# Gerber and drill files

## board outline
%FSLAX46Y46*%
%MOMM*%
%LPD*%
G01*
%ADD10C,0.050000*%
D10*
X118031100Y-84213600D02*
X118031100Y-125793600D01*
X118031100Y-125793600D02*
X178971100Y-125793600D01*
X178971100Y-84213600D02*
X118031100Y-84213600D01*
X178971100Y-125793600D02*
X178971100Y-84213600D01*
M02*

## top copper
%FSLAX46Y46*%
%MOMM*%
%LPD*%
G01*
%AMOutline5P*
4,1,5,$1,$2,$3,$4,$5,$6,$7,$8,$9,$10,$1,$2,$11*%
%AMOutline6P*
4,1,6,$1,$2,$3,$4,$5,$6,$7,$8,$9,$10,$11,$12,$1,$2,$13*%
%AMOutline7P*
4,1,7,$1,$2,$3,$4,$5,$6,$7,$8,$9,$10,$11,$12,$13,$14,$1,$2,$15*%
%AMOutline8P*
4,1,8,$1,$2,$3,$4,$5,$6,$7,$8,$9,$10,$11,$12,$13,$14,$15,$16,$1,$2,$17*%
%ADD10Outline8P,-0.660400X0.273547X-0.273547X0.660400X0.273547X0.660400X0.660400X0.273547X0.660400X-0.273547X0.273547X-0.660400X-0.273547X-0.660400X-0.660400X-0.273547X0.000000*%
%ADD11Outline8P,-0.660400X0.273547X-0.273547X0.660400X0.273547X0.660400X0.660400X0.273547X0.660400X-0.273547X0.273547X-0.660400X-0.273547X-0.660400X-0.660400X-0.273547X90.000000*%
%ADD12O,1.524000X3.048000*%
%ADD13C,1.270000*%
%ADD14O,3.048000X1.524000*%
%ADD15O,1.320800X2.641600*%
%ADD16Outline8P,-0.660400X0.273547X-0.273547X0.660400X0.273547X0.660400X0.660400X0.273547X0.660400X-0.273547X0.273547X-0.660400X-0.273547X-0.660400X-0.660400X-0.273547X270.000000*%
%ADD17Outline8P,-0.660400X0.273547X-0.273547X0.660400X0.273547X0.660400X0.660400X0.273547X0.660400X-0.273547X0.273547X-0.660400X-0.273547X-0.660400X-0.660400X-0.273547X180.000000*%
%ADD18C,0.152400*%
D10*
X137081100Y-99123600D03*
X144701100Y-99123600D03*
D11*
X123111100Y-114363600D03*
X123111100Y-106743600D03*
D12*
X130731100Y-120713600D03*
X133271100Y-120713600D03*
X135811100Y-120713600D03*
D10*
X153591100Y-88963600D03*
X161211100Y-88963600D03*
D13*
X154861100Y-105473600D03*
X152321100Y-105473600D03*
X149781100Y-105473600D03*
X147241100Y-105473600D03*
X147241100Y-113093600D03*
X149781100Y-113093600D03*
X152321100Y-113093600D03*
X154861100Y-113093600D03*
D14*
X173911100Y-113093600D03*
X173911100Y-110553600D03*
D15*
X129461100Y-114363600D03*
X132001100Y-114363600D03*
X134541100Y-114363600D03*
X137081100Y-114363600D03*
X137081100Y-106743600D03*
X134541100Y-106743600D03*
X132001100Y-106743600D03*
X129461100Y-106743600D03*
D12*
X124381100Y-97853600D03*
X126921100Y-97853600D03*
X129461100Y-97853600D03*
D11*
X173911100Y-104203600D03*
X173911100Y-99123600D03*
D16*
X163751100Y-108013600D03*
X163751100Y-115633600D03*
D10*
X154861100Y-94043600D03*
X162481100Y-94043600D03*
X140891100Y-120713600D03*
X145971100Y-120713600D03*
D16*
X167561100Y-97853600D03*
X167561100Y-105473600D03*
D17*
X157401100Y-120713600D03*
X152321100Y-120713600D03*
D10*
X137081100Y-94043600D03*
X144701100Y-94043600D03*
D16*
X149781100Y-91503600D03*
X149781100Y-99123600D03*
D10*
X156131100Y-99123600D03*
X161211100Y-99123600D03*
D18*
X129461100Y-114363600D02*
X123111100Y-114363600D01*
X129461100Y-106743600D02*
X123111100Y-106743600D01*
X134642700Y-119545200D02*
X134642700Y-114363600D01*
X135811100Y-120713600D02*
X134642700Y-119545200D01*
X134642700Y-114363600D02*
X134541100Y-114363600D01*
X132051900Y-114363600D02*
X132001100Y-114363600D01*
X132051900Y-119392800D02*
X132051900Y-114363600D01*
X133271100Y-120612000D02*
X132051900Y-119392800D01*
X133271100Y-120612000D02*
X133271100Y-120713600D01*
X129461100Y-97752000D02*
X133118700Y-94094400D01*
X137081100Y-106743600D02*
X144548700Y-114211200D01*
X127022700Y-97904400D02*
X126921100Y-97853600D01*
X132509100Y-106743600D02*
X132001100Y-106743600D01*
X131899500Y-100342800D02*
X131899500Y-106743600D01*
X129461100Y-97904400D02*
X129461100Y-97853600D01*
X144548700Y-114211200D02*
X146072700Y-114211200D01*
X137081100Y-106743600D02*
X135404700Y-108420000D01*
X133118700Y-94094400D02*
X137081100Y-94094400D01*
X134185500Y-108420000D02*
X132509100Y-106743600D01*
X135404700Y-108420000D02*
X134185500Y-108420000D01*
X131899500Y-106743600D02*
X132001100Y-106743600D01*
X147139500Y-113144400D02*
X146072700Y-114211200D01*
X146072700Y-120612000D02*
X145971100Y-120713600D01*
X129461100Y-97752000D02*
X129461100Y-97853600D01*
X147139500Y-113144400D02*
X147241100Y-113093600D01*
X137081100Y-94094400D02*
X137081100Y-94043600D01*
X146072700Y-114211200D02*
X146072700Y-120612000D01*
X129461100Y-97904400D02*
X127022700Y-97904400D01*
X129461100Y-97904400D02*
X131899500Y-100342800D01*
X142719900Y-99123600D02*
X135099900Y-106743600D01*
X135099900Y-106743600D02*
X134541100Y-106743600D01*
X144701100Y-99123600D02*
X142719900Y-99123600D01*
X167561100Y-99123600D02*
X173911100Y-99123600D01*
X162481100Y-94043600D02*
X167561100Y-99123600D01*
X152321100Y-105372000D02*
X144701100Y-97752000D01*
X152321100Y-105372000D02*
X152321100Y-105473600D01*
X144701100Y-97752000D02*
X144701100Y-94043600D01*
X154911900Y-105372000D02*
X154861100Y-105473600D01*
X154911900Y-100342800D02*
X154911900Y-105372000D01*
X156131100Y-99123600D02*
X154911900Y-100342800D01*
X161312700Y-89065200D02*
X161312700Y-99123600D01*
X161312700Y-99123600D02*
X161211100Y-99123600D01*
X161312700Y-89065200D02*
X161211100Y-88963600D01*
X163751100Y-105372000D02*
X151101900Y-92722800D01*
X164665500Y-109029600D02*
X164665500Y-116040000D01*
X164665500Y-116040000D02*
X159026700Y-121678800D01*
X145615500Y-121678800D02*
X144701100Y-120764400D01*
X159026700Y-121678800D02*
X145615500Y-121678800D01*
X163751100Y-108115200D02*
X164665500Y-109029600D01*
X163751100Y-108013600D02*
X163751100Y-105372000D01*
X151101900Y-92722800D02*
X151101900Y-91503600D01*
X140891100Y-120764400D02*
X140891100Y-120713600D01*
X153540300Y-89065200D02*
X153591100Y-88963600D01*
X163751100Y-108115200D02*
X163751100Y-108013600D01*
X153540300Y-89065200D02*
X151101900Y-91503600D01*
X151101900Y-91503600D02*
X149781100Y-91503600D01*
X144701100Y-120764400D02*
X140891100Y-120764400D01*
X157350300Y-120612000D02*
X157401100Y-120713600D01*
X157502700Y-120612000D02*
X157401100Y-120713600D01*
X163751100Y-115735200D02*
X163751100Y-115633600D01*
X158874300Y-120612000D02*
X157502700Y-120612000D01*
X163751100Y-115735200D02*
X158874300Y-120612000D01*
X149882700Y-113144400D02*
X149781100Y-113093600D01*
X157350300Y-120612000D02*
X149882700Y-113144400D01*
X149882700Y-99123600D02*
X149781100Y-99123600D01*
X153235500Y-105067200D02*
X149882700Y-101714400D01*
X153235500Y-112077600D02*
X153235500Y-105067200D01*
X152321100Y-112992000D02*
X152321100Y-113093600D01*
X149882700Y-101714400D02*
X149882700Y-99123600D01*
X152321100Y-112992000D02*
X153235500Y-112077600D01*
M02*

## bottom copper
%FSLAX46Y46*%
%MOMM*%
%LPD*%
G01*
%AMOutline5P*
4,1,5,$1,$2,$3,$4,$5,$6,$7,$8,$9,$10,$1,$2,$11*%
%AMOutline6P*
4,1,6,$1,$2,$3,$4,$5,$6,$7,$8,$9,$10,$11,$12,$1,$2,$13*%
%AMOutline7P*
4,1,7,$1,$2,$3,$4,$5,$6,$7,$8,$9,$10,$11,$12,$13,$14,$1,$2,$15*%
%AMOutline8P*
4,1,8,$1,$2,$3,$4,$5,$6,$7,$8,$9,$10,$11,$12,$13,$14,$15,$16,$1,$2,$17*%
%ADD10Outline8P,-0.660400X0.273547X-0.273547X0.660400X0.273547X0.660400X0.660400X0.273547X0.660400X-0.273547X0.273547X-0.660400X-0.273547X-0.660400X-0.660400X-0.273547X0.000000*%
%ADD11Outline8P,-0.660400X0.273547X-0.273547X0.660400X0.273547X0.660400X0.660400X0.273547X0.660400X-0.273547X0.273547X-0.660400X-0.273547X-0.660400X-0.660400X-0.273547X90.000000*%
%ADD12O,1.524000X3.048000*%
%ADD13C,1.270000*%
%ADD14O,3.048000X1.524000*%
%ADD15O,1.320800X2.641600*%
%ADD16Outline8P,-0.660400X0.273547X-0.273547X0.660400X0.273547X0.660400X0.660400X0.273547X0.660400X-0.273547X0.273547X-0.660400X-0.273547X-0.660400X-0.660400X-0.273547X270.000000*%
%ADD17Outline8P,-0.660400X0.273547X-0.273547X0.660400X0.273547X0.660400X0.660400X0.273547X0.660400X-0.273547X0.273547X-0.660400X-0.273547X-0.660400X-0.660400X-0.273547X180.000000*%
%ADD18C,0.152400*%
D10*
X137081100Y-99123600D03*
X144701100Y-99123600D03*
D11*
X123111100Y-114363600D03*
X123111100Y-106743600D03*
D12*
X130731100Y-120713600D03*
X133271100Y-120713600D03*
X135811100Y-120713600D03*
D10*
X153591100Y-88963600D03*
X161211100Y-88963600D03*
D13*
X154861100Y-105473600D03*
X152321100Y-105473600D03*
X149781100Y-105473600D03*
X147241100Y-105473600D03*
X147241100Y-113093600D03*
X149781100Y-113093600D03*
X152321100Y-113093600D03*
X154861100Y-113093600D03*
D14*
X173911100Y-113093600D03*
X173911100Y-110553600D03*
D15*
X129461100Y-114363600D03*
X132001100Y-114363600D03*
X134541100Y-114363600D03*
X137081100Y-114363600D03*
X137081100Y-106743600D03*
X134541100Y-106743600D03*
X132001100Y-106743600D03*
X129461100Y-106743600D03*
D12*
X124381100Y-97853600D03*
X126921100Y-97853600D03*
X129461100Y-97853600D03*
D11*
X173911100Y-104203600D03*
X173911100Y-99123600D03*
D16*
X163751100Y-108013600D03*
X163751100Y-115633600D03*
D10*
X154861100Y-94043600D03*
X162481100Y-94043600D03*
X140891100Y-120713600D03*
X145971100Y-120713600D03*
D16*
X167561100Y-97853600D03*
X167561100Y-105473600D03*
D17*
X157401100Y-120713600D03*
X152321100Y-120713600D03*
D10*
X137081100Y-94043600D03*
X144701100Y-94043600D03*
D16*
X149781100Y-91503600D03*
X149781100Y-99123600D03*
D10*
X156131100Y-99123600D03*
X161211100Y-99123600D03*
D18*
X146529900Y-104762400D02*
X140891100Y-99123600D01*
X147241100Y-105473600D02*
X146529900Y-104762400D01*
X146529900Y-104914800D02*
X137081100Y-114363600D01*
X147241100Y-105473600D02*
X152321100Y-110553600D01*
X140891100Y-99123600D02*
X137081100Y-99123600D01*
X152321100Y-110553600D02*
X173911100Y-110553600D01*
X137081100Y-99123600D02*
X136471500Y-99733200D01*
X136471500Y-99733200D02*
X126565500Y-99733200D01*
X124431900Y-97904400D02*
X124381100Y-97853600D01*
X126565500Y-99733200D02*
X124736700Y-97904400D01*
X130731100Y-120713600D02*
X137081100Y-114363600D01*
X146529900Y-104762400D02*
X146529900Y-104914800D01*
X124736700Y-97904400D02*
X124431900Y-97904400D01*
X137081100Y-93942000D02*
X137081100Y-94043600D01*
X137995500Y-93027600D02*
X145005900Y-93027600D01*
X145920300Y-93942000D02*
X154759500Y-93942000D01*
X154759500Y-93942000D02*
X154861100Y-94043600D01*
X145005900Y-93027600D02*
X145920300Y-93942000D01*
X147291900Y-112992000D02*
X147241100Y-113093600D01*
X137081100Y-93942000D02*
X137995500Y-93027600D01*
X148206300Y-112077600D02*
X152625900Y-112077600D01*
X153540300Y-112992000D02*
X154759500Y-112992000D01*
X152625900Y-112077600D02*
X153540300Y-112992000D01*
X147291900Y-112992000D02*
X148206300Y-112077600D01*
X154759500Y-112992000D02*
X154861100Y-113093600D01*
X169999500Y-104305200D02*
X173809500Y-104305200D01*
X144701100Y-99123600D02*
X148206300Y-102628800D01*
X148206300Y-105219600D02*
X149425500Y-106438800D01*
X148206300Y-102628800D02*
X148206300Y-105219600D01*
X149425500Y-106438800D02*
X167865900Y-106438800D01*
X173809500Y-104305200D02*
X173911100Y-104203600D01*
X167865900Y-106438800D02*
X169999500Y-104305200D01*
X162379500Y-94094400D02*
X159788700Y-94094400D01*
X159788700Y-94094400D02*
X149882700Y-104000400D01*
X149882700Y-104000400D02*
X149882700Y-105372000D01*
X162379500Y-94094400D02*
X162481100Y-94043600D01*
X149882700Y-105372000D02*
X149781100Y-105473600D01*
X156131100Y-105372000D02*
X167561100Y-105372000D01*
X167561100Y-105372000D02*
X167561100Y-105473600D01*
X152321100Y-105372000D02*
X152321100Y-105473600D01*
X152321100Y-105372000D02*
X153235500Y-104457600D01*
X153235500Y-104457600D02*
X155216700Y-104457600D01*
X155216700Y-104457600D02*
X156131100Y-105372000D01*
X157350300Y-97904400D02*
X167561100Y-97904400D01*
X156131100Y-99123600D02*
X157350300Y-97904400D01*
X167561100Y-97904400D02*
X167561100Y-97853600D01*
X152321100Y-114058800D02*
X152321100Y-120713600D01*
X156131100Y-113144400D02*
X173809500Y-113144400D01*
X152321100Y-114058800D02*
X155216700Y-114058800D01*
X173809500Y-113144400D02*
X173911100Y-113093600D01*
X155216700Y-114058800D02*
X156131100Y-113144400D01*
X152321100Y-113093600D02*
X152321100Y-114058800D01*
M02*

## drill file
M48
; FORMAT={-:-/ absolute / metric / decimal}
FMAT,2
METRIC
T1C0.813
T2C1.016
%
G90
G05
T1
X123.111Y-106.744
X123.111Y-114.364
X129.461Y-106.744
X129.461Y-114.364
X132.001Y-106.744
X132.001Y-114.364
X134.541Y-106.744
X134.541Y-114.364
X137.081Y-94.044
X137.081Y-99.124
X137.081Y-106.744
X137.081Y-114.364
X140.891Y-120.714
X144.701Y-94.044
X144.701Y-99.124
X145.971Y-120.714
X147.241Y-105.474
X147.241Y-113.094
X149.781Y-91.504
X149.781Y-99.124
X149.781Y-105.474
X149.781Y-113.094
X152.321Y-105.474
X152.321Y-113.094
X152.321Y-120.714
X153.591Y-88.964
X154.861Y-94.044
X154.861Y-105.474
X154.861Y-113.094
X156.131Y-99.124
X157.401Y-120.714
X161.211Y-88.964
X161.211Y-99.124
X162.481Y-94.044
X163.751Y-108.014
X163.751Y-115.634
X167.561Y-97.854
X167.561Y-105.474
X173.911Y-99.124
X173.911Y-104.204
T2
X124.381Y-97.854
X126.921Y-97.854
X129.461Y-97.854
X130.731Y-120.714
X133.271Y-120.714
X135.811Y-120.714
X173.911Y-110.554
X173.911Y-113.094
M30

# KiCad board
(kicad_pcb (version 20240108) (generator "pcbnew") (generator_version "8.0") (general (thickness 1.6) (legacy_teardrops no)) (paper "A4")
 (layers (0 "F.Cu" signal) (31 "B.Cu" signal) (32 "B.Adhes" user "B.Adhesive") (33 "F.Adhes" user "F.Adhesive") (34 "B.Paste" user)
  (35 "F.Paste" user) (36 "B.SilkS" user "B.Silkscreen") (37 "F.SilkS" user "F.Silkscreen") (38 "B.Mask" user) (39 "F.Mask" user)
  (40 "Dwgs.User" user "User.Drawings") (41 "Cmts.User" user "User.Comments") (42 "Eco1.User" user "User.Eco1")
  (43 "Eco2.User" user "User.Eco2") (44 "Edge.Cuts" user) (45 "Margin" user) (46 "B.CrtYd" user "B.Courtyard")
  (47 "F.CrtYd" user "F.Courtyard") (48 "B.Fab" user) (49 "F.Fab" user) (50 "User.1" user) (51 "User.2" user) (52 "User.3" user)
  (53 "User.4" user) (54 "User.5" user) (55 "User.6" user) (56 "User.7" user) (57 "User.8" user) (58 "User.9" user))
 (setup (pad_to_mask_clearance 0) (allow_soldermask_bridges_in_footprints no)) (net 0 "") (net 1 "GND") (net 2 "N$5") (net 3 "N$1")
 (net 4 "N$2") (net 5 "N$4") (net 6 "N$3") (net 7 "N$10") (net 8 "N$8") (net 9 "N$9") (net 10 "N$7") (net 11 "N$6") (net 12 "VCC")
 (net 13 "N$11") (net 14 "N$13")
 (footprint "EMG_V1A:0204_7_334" (layer "F.Cu") (at 140.8911 99.1236)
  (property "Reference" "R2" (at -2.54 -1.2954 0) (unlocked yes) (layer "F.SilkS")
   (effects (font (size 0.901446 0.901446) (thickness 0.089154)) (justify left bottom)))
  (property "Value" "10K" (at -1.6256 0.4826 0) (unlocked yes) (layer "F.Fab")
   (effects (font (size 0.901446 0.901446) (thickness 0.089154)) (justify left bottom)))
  (pad "1" thru_hole roundrect (at -3.81 0) (size 1.3208 1.3208) (drill 0.8128) (layers "*.Cu" "*.Mask") (remove_unused_layers no)
   (roundrect_rratio 0.25) (chamfer_ratio 0.2928932188) (chamfer top_left top_right bottom_left bottom_right) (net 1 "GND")
   (solder_mask_margin 0.1016) (thermal_bridge_angle 0))
  (pad "2" thru_hole roundrect (at 3.81 0) (size 1.3208 1.3208) (drill 0.8128) (layers "*.Cu" "*.Mask") (remove_unused_layers no)
   (roundrect_rratio 0.25) (chamfer_ratio 0.2928932188) (chamfer top_left top_right bottom_left bottom_right) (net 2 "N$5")
   (solder_mask_margin 0.1016) (thermal_bridge_angle 0)))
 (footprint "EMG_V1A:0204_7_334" (layer "F.Cu") (at 123.1111 110.5536 90)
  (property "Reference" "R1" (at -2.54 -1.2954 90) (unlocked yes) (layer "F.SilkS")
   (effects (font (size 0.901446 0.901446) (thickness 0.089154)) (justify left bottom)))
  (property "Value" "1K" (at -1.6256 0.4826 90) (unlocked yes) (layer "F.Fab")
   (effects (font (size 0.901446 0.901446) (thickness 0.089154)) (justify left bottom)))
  (pad "1" thru_hole roundrect (at -3.81 0 90) (size 1.3208 1.3208) (drill 0.8128) (layers "*.Cu" "*.Mask") (remove_unused_layers no)
   (roundrect_rratio 0.25) (chamfer_ratio 0.2928932188) (chamfer top_left top_right bottom_left bottom_right) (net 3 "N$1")
   (solder_mask_margin 0.1016) (thermal_bridge_angle 0))
  (pad "2" thru_hole roundrect (at 3.81 0 90) (size 1.3208 1.3208) (drill 0.8128) (layers "*.Cu" "*.Mask") (remove_unused_layers no)
   (roundrect_rratio 0.25) (chamfer_ratio 0.2928932188) (chamfer top_left top_right bottom_left bottom_right) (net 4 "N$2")
   (solder_mask_margin 0.1016) (thermal_bridge_angle 0)))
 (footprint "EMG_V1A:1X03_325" (layer "F.Cu") (at 133.2711 120.7136)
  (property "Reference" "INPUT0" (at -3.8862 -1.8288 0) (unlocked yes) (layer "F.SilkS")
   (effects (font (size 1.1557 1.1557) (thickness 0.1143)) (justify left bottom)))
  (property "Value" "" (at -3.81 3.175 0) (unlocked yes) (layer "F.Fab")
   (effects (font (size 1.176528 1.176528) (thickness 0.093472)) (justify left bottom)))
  (pad "1" thru_hole oval (at -2.54 0 90) (size 3.048 1.524) (drill 1.016) (layers "*.Cu" "*.Mask") (remove_unused_layers no) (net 1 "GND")
   (solder_mask_margin 0.1016) (thermal_bridge_angle 0))
  (pad "2" thru_hole oval (at 0 0 90) (size 3.048 1.524) (drill 1.016) (layers "*.Cu" "*.Mask") (remove_unused_layers no) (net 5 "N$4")
   (solder_mask_margin 0.1016) (thermal_bridge_angle 0))
  (pad "3" thru_hole oval (at 2.54 0 90) (size 3.048 1.524) (drill 1.016) (layers "*.Cu" "*.Mask") (remove_unused_layers no) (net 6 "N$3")
   (solder_mask_margin 0.1016) (thermal_bridge_angle 0)))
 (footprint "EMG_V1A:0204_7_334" (layer "F.Cu") (at 157.4011 88.9636)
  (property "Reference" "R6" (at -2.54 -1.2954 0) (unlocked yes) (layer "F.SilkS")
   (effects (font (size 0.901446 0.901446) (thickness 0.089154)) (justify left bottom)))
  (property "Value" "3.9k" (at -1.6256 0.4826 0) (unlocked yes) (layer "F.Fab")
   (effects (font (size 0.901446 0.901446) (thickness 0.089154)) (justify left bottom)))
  (pad "1" thru_hole roundrect (at -3.81 0) (size 1.3208 1.3208) (drill 0.8128) (layers "*.Cu" "*.Mask") (remove_unused_layers no)
   (roundrect_rratio 0.25) (chamfer_ratio 0.2928932188) (chamfer top_left top_right bottom_left bottom_right) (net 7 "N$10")
   (solder_mask_margin 0.1016) (thermal_bridge_angle 0))
  (pad "2" thru_hole roundrect (at 3.81 0) (size 1.3208 1.3208) (drill 0.8128) (layers "*.Cu" "*.Mask") (remove_unused_layers no)
   (roundrect_rratio 0.25) (chamfer_ratio 0.2928932188) (chamfer top_left top_right bottom_left bottom_right) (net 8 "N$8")
   (solder_mask_margin 0.1016) (thermal_bridge_angle 0)))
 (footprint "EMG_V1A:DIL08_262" (layer "F.Cu") (at 151.0511 109.2836 180)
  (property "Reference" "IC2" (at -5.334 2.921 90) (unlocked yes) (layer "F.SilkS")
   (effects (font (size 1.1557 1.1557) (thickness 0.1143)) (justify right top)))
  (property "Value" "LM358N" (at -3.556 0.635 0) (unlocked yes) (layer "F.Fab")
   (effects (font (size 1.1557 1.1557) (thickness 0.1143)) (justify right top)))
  (pad "1" thru_hole circle (at -3.81 3.81 270) (size 1.27 1.27) (drill 0.8128) (layers "*.Cu" "*.Mask") (remove_unused_layers no)
   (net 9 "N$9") (solder_mask_margin 0.1016) (thermal_bridge_angle 0))
  (pad "2" thru_hole circle (at -1.27 3.81 270) (size 1.27 1.27) (drill 0.8128) (layers "*.Cu" "*.Mask") (remove_unused_layers no)
   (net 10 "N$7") (solder_mask_margin 0.1016) (thermal_bridge_angle 0))
  (pad "3" thru_hole circle (at 1.27 3.81 270) (size 1.27 1.27) (drill 0.8128) (layers "*.Cu" "*.Mask") (remove_unused_layers no)
   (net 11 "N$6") (solder_mask_margin 0.1016) (thermal_bridge_angle 0))
  (pad "4" thru_hole circle (at 3.81 3.81 270) (size 1.27 1.27) (drill 0.8128) (layers "*.Cu" "*.Mask") (remove_unused_layers no)
   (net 1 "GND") (solder_mask_margin 0.1016) (thermal_bridge_angle 0))
  (pad "5" thru_hole circle (at 3.81 -3.81 270) (size 1.27 1.27) (drill 0.8128) (layers "*.Cu" "*.Mask") (remove_unused_layers no)
   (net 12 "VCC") (solder_mask_margin 0.1016) (thermal_bridge_angle 0))
  (pad "6" thru_hole circle (at 1.27 -3.81 270) (size 1.27 1.27) (drill 0.8128) (layers "*.Cu" "*.Mask") (remove_unused_layers no)
   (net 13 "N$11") (solder_mask_margin 0.1016) (thermal_bridge_angle 0))
  (pad "7" thru_hole circle (at -1.27 -3.81 270) (size 1.27 1.27) (drill 0.8128) (layers "*.Cu" "*.Mask") (remove_unused_layers no)
   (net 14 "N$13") (solder_mask_margin 0.1016) (thermal_bridge_angle 0))
  (pad "8" thru_hole circle (at -3.81 -3.81 270) (size 1.27 1.27) (drill 0.8128) (layers "*.Cu" "*.Mask") (remove_unused_layers no)
   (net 12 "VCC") (solder_mask_margin 0.1016) (thermal_bridge_angle 0)))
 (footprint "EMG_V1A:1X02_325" (layer "F.Cu") (at 173.9111 111.8236 90)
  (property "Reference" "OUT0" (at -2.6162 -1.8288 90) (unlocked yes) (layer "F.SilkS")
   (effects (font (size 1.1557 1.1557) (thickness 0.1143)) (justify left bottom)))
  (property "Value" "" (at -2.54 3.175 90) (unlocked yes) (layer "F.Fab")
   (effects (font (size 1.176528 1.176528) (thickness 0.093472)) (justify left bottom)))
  (pad "1" thru_hole oval (at -1.27 0 180) (size 3.048 1.524) (drill 1.016) (layers "*.Cu" "*.Mask") (remove_unused_layers no)
   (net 14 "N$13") (solder_mask_margin 0.1016) (thermal_bridge_angle 0))
  (pad "2" thru_hole oval (at 1.27 0 180) (size 3.048 1.524) (drill 1.016) (layers "*.Cu" "*.Mask") (remove_unused_layers no) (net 1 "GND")
   (solder_mask_margin 0.1016) (thermal_bridge_angle 0)))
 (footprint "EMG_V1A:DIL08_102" (layer "F.Cu") (at 133.2711 110.5536)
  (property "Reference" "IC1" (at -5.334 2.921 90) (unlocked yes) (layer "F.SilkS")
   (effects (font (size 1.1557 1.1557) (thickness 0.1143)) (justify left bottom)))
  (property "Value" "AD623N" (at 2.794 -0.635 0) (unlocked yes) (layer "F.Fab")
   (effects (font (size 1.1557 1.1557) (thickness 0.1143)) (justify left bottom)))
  (pad "1" thru_hole oval (at -3.81 3.81 90) (size 2.6416 1.3208) (drill 0.8128) (layers "*.Cu" "*.Mask") (remove_unused_layers no)
   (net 3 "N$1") (solder_mask_margin 0.1016) (thermal_bridge_angle 0))
  (pad "2" thru_hole oval (at -1.27 3.81 90) (size 2.6416 1.3208) (drill 0.8128) (layers "*.Cu" "*.Mask") (remove_unused_layers no)
   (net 5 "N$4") (solder_mask_margin 0.1016) (thermal_bridge_angle 0))
  (pad "3" thru_hole oval (at 1.27 3.81 90) (size 2.6416 1.3208) (drill 0.8128) (layers "*.Cu" "*.Mask") (remove_unused_layers no)
   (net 6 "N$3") (solder_mask_margin 0.1016) (thermal_bridge_angle 0))
  (pad "4" thru_hole oval (at 3.81 3.81 90) (size 2.6416 1.3208) (drill 0.8128) (layers "*.Cu" "*.Mask") (remove_unused_layers no)
   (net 1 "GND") (solder_mask_margin 0.1016) (thermal_bridge_angle 0))
  (pad "5" thru_hole oval (at 3.81 -3.81 90) (size 2.6416 1.3208) (drill 0.8128) (layers "*.Cu" "*.Mask") (remove_unused_layers no)
   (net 12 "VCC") (solder_mask_margin 0.1016) (thermal_bridge_angle 0))
  (pad "6" thru_hole oval (at 1.27 -3.81 90) (size 2.6416 1.3208) (drill 0.8128) (layers "*.Cu" "*.Mask") (remove_unused_layers no)
   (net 2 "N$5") (solder_mask_margin 0.1016) (thermal_bridge_angle 0))
  (pad "7" thru_hole oval (at -1.27 -3.81 90) (size 2.6416 1.3208) (drill 0.8128) (layers "*.Cu" "*.Mask") (remove_unused_layers no)
   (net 12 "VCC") (solder_mask_margin 0.1016) (thermal_bridge_angle 0))
  (pad "8" thru_hole oval (at -3.81 -3.81 90) (size 2.6416 1.3208) (drill 0.8128) (layers "*.Cu" "*.Mask") (remove_unused_layers no)
   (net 4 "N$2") (solder_mask_margin 0.1016) (thermal_bridge_angle 0)))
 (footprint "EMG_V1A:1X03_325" (layer "F.Cu") (at 126.9211 97.8536)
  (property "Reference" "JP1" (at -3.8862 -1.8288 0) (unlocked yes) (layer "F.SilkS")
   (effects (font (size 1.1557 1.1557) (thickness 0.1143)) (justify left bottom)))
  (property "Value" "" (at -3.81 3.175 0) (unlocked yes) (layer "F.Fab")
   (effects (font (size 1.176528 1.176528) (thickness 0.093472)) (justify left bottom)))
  (pad "1" thru_hole oval (at -2.54 0 90) (size 3.048 1.524) (drill 1.016) (layers "*.Cu" "*.Mask") (remove_unused_layers no) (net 1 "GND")
   (solder_mask_margin 0.1016) (thermal_bridge_angle 0))
  (pad "2" thru_hole oval (at 0 0 90) (size 3.048 1.524) (drill 1.016) (layers "*.Cu" "*.Mask") (remove_unused_layers no) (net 12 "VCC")
   (solder_mask_margin 0.1016) (thermal_bridge_angle 0))
  (pad "3" thru_hole oval (at 2.54 0 90) (size 3.048 1.524) (drill 1.016) (layers "*.Cu" "*.Mask") (remove_unused_layers no) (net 12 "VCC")
   (solder_mask_margin 0.1016) (thermal_bridge_angle 0)))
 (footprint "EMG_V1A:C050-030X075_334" (layer "F.Cu") (at 173.9111 101.6636 90)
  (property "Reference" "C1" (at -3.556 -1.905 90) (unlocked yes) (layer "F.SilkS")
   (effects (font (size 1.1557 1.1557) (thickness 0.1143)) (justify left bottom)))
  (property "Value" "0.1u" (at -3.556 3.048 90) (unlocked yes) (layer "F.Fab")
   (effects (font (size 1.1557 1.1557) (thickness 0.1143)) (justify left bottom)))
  (pad "1" thru_hole roundrect (at -2.54 0 90) (size 1.3208 1.3208) (drill 0.8128) (layers "*.Cu" "*.Mask") (remove_unused_layers no)
   (roundrect_rratio 0.25) (chamfer_ratio 0.2928932188) (chamfer top_left top_right bottom_left bottom_right) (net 2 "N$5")
   (solder_mask_margin 0.1016) (thermal_bridge_angle 0))
  (pad "2" thru_hole roundrect (at 2.54 0 90) (size 1.3208 1.3208) (drill 0.8128) (layers "*.Cu" "*.Mask") (remove_unused_layers no)
   (roundrect_rratio 0.25) (chamfer_ratio 0.2928932188) (chamfer top_left top_right bottom_left bottom_right) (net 11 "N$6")
   (solder_mask_margin 0.1016) (thermal_bridge_angle 0)))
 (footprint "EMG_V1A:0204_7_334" (layer "F.Cu") (at 163.7511 111.8236 -90)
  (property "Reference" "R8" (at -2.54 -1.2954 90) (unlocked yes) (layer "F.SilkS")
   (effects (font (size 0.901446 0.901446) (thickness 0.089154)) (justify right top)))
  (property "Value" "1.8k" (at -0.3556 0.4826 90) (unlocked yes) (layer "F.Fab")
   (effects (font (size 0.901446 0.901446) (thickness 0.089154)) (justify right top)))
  (pad "1" thru_hole roundrect (at -3.81 0 270) (size 1.3208 1.3208) (drill 0.8128) (layers "*.Cu" "*.Mask") (remove_unused_layers no)
   (roundrect_rratio 0.25) (chamfer_ratio 0.2928932188) (chamfer top_left top_right bottom_left bottom_right) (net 7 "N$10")
   (solder_mask_margin 0.1016) (thermal_bridge_angle 0))
  (pad "2" thru_hole roundrect (at 3.81 0 270) (size 1.3208 1.3208) (drill 0.8128) (layers "*.Cu" "*.Mask") (remove_unused_layers no)
   (roundrect_rratio 0.25) (chamfer_ratio 0.2928932188) (chamfer top_left top_right bottom_left bottom_right) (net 13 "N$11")
   (solder_mask_margin 0.1016) (thermal_bridge_angle 0)))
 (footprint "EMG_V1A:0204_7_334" (layer "F.Cu") (at 158.6711 94.0436)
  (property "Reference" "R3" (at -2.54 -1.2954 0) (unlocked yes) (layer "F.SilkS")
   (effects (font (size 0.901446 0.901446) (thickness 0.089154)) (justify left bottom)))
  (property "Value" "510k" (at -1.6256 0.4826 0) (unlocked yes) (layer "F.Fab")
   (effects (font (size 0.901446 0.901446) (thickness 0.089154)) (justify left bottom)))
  (pad "1" thru_hole roundrect (at -3.81 0) (size 1.3208 1.3208) (drill 0.8128) (layers "*.Cu" "*.Mask") (remove_unused_layers no)
   (roundrect_rratio 0.25) (chamfer_ratio 0.2928932188) (chamfer top_left top_right bottom_left bottom_right) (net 12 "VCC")
   (solder_mask_margin 0.1016) (thermal_bridge_angle 0))
  (pad "2" thru_hole roundrect (at 3.81 0) (size 1.3208 1.3208) (drill 0.8128) (layers "*.Cu" "*.Mask") (remove_unused_layers no)
   (roundrect_rratio 0.25) (chamfer_ratio 0.2928932188) (chamfer top_left top_right bottom_left bottom_right) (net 11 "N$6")
   (solder_mask_margin 0.1016) (thermal_bridge_angle 0)))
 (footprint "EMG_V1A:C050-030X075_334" (layer "F.Cu") (at 143.4311 120.7136)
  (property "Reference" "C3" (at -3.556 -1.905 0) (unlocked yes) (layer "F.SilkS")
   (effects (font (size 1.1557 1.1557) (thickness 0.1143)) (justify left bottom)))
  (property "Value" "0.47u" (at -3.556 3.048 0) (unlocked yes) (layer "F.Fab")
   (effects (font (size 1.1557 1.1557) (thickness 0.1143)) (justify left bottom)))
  (pad "1" thru_hole roundrect (at -2.54 0) (size 1.3208 1.3208) (drill 0.8128) (layers "*.Cu" "*.Mask") (remove_unused_layers no)
   (roundrect_rratio 0.25) (chamfer_ratio 0.2928932188) (chamfer top_left top_right bottom_left bottom_right) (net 7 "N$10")
   (solder_mask_margin 0.1016) (thermal_bridge_angle 0))
  (pad "2" thru_hole roundrect (at 2.54 0) (size 1.3208 1.3208) (drill 0.8128) (layers "*.Cu" "*.Mask") (remove_unused_layers no)
   (roundrect_rratio 0.25) (chamfer_ratio 0.2928932188) (chamfer top_left top_right bottom_left bottom_right) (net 12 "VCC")
   (solder_mask_margin 0.1016) (thermal_bridge_angle 0)))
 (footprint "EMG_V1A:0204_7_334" (layer "F.Cu") (at 167.5611 101.6636 -90)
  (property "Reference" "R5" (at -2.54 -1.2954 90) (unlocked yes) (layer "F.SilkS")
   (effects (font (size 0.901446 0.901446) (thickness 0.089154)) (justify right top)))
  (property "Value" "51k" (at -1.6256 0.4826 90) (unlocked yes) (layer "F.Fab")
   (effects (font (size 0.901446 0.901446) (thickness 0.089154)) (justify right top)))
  (pad "1" thru_hole roundrect (at -3.81 0 270) (size 1.3208 1.3208) (drill 0.8128) (layers "*.Cu" "*.Mask") (remove_unused_layers no)
   (roundrect_rratio 0.25) (chamfer_ratio 0.2928932188) (chamfer top_left top_right bottom_left bottom_right) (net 9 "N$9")
   (solder_mask_margin 0.1016) (thermal_bridge_angle 0))
  (pad "2" thru_hole roundrect (at 3.81 0 270) (size 1.3208 1.3208) (drill 0.8128) (layers "*.Cu" "*.Mask") (remove_unused_layers no)
   (roundrect_rratio 0.25) (chamfer_ratio 0.2928932188) (chamfer top_left top_right bottom_left bottom_right) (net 10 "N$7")
   (solder_mask_margin 0.1016) (thermal_bridge_angle 0)))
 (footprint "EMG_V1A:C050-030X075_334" (layer "F.Cu") (at 154.8611 120.7136 180)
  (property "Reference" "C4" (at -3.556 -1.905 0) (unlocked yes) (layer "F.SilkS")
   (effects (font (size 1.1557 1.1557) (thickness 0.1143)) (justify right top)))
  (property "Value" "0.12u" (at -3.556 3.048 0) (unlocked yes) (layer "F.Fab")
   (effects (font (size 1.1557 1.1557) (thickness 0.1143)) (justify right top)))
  (pad "1" thru_hole roundrect (at -2.54 0 180) (size 1.3208 1.3208) (drill 0.8128) (layers "*.Cu" "*.Mask") (remove_unused_layers no)
   (roundrect_rratio 0.25) (chamfer_ratio 0.2928932188) (chamfer top_left top_right bottom_left bottom_right) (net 13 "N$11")
   (solder_mask_margin 0.1016) (thermal_bridge_angle 0))
  (pad "2" thru_hole roundrect (at 2.54 0 180) (size 1.3208 1.3208) (drill 0.8128) (layers "*.Cu" "*.Mask") (remove_unused_layers no)
   (roundrect_rratio 0.25) (chamfer_ratio 0.2928932188) (chamfer top_left top_right bottom_left bottom_right) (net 14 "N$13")
   (solder_mask_margin 0.1016) (thermal_bridge_angle 0)))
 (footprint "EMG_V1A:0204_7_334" (layer "F.Cu") (at 140.8911 94.0436)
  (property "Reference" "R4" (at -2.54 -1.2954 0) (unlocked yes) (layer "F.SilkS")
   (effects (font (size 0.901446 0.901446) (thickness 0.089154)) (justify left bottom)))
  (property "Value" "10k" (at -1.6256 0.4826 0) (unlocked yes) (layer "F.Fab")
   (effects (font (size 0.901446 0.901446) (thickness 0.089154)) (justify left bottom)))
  (pad "1" thru_hole roundrect (at -3.81 0) (size 1.3208 1.3208) (drill 0.8128) (layers "*.Cu" "*.Mask") (remove_unused_layers no)
   (roundrect_rratio 0.25) (chamfer_ratio 0.2928932188) (chamfer top_left top_right bottom_left bottom_right) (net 12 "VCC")
   (solder_mask_margin 0.1016) (thermal_bridge_angle 0))
  (pad "2" thru_hole roundrect (at 3.81 0) (size 1.3208 1.3208) (drill 0.8128) (layers "*.Cu" "*.Mask") (remove_unused_layers no)
   (roundrect_rratio 0.25) (chamfer_ratio 0.2928932188) (chamfer top_left top_right bottom_left bottom_right) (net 10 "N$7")
   (solder_mask_margin 0.1016) (thermal_bridge_angle 0)))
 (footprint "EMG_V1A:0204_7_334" (layer "F.Cu") (at 149.7811 95.3136 -90)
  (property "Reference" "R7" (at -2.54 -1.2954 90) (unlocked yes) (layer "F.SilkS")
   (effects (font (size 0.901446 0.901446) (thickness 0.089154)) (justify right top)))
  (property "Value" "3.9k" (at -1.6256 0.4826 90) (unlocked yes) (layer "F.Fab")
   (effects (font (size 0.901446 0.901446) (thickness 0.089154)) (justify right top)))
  (pad "1" thru_hole roundrect (at -3.81 0 270) (size 1.3208 1.3208) (drill 0.8128) (layers "*.Cu" "*.Mask") (remove_unused_layers no)
   (roundrect_rratio 0.25) (chamfer_ratio 0.2928932188) (chamfer top_left top_right bottom_left bottom_right) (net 7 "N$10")
   (solder_mask_margin 0.1016) (thermal_bridge_angle 0))
  (pad "2" thru_hole roundrect (at 3.81 0 270) (size 1.3208 1.3208) (drill 0.8128) (layers "*.Cu" "*.Mask") (remove_unused_layers no)
   (roundrect_rratio 0.25) (chamfer_ratio 0.2928932188) (chamfer top_left top_right bottom_left bottom_right) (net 14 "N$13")
   (solder_mask_margin 0.1016) (thermal_bridge_angle 0)))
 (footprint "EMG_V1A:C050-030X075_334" (layer "F.Cu") (at 158.6711 99.1236)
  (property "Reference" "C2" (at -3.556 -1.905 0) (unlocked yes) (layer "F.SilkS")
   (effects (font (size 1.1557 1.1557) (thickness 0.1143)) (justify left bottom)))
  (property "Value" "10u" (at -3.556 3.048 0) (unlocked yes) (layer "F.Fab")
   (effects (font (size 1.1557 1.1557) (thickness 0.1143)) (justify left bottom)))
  (pad "1" thru_hole roundrect (at -2.54 0) (size 1.3208 1.3208) (drill 0.8128) (layers "*.Cu" "*.Mask") (remove_unused_layers no)
   (roundrect_rratio 0.25) (chamfer_ratio 0.2928932188) (chamfer top_left top_right bottom_left bottom_right) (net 9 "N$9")
   (solder_mask_margin 0.1016) (thermal_bridge_angle 0))
  (pad "2" thru_hole roundrect (at 2.54 0) (size 1.3208 1.3208) (drill 0.8128) (layers "*.Cu" "*.Mask") (remove_unused_layers no)
   (roundrect_rratio 0.25) (chamfer_ratio 0.2928932188) (chamfer top_left top_right bottom_left bottom_right) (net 8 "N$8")
   (solder_mask_margin 0.1016) (thermal_bridge_angle 0)))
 (gr_line (start 118.0311 84.2136) (end 118.0311 125.7936) (stroke (width 0.05) (type solid)) (layer "Edge.Cuts"))
 (gr_line (start 118.0311 125.7936) (end 178.9711 125.7936) (stroke (width 0.05) (type solid)) (layer "Edge.Cuts"))
 (gr_line (start 178.9711 84.2136) (end 118.0311 84.2136) (stroke (width 0.05) (type solid)) (layer "Edge.Cuts"))
 (gr_line (start 178.9711 125.7936) (end 178.9711 84.2136) (stroke (width 0.05) (type solid)) (layer "Edge.Cuts"))
 (segment (start 129.4611 114.3636) (end 123.1111 114.3636) (width 0.1524) (layer "F.Cu") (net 3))
 (segment (start 129.4611 106.7436) (end 123.1111 106.7436) (width 0.1524) (layer "F.Cu") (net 4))
 (segment (start 134.6427 119.5452) (end 134.6427 114.3636) (width 0.1524) (layer "F.Cu") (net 6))
 (segment (start 135.8111 120.7136) (end 134.6427 119.5452) (width 0.1524) (layer "F.Cu") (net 6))
 (segment (start 134.6427 114.3636) (end 134.5411 114.3636) (width 0.1524) (layer "F.Cu") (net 6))
 (segment (start 132.0519 114.3636) (end 132.0011 114.3636) (width 0.1524) (layer "F.Cu") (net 5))
 (segment (start 132.0519 119.3928) (end 132.0519 114.3636) (width 0.1524) (layer "F.Cu") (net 5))
 (segment (start 133.2711 120.612) (end 132.0519 119.3928) (width 0.1524) (layer "F.Cu") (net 5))
 (segment (start 133.2711 120.612) (end 133.2711 120.7136) (width 0.1524) (layer "F.Cu") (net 5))
 (segment (start 146.5299 104.7624) (end 140.8911 99.1236) (width 0.1524) (layer "B.Cu") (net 1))
 (segment (start 147.2411 105.4736) (end 146.5299 104.7624) (width 0.1524) (layer "B.Cu") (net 1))
 (segment (start 146.5299 104.9148) (end 137.0811 114.3636) (width 0.1524) (layer "B.Cu") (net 1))
 (segment (start 147.2411 105.4736) (end 152.3211 110.5536) (width 0.1524) (layer "B.Cu") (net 1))
 (segment (start 140.8911 99.1236) (end 137.0811 99.1236) (width 0.1524) (layer "B.Cu") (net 1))
 (segment (start 152.3211 110.5536) (end 173.9111 110.5536) (width 0.1524) (layer "B.Cu") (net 1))
 (segment (start 137.0811 99.1236) (end 136.4715 99.7332) (width 0.1524) (layer "B.Cu") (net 1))
 (segment (start 136.4715 99.7332) (end 126.5655 99.7332) (width 0.1524) (layer "B.Cu") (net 1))
 (segment (start 124.4319 97.9044) (end 124.3811 97.8536) (width 0.1524) (layer "B.Cu") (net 1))
 (segment (start 126.5655 99.7332) (end 124.7367 97.9044) (width 0.1524) (layer "B.Cu") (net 1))
 (segment (start 130.7311 120.7136) (end 137.0811 114.3636) (width 0.1524) (layer "B.Cu") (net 1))
 (segment (start 146.5299 104.7624) (end 146.5299 104.9148) (width 0.1524) (layer "B.Cu") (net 1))
 (segment (start 124.7367 97.9044) (end 124.4319 97.9044) (width 0.1524) (layer "B.Cu") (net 1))
 (segment (start 129.4611 97.752) (end 133.1187 94.0944) (width 0.1524) (layer "F.Cu") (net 12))
 (segment (start 137.0811 106.7436) (end 144.5487 114.2112) (width 0.1524) (layer "F.Cu") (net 12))
 (segment (start 127.0227 97.9044) (end 126.9211 97.8536) (width 0.1524) (layer "F.Cu") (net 12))
 (segment (start 132.5091 106.7436) (end 132.0011 106.7436) (width 0.1524) (layer "F.Cu") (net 12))
 (segment (start 131.8995 100.3428) (end 131.8995 106.7436) (width 0.1524) (layer "F.Cu") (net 12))
 (segment (start 129.4611 97.9044) (end 129.4611 97.8536) (width 0.1524) (layer "F.Cu") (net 12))
 (segment (start 144.5487 114.2112) (end 146.0727 114.2112) (width 0.1524) (layer "F.Cu") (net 12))
 (segment (start 137.0811 106.7436) (end 135.4047 108.42) (width 0.1524) (layer "F.Cu") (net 12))
 (segment (start 133.1187 94.0944) (end 137.0811 94.0944) (width 0.1524) (layer "F.Cu") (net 12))
 (segment (start 134.1855 108.42) (end 132.5091 106.7436) (width 0.1524) (layer "F.Cu") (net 12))
 (segment (start 135.4047 108.42) (end 134.1855 108.42) (width 0.1524) (layer "F.Cu") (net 12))
 (segment (start 131.8995 106.7436) (end 132.0011 106.7436) (width 0.1524) (layer "F.Cu") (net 12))
 (segment (start 147.1395 113.1444) (end 146.0727 114.2112) (width 0.1524) (layer "F.Cu") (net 12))
 (segment (start 146.0727 120.612) (end 145.9711 120.7136) (width 0.1524) (layer "F.Cu") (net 12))
 (segment (start 129.4611 97.752) (end 129.4611 97.8536) (width 0.1524) (layer "F.Cu") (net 12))
 (segment (start 147.1395 113.1444) (end 147.2411 113.0936) (width 0.1524) (layer "F.Cu") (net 12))
 (segment (start 137.0811 94.0944) (end 137.0811 94.0436) (width 0.1524) (layer "F.Cu") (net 12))
 (segment (start 146.0727 114.2112) (end 146.0727 120.612) (width 0.1524) (layer "F.Cu") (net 12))
 (segment (start 129.4611 97.9044) (end 127.0227 97.9044) (width 0.1524) (layer "F.Cu") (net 12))
 (segment (start 129.4611 97.9044) (end 131.8995 100.3428) (width 0.1524) (layer "F.Cu") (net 12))
 (segment (start 137.0811 93.942) (end 137.0811 94.0436) (width 0.1524) (layer "B.Cu") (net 12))
 (segment (start 137.9955 93.0276) (end 145.0059 93.0276) (width 0.1524) (layer "B.Cu") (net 12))
 (segment (start 145.9203 93.942) (end 154.7595 93.942) (width 0.1524) (layer "B.Cu") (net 12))
 (segment (start 154.7595 93.942) (end 154.8611 94.0436) (width 0.1524) (layer "B.Cu") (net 12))
 (segment (start 145.0059 93.0276) (end 145.9203 93.942) (width 0.1524) (layer "B.Cu") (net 12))
 (segment (start 147.2919 112.992) (end 147.2411 113.0936) (width 0.1524) (layer "B.Cu") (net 12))
 (segment (start 137.0811 93.942) (end 137.9955 93.0276) (width 0.1524) (layer "B.Cu") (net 12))
 (segment (start 148.2063 112.0776) (end 152.6259 112.0776) (width 0.1524) (layer "B.Cu") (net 12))
 (segment (start 153.5403 112.992) (end 154.7595 112.992) (width 0.1524) (layer "B.Cu") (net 12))
 (segment (start 152.6259 112.0776) (end 153.5403 112.992) (width 0.1524) (layer "B.Cu") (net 12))
 (segment (start 147.2919 112.992) (end 148.2063 112.0776) (width 0.1524) (layer "B.Cu") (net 12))
 (segment (start 154.7595 112.992) (end 154.8611 113.0936) (width 0.1524) (layer "B.Cu") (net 12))
 (segment (start 142.7199 99.1236) (end 135.0999 106.7436) (width 0.1524) (layer "F.Cu") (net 2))
 (segment (start 135.0999 106.7436) (end 134.5411 106.7436) (width 0.1524) (layer "F.Cu") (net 2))
 (segment (start 144.7011 99.1236) (end 142.7199 99.1236) (width 0.1524) (layer "F.Cu") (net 2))
 (segment (start 169.9995 104.3052) (end 173.8095 104.3052) (width 0.1524) (layer "B.Cu") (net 2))
 (segment (start 144.7011 99.1236) (end 148.2063 102.6288) (width 0.1524) (layer "B.Cu") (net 2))
 (segment (start 148.2063 105.2196) (end 149.4255 106.4388) (width 0.1524) (layer "B.Cu") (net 2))
 (segment (start 148.2063 102.6288) (end 148.2063 105.2196) (width 0.1524) (layer "B.Cu") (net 2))
 (segment (start 149.4255 106.4388) (end 167.8659 106.4388) (width 0.1524) (layer "B.Cu") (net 2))
 (segment (start 173.8095 104.3052) (end 173.9111 104.2036) (width 0.1524) (layer "B.Cu") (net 2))
 (segment (start 167.8659 106.4388) (end 169.9995 104.3052) (width 0.1524) (layer "B.Cu") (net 2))
 (segment (start 167.5611 99.1236) (end 173.9111 99.1236) (width 0.1524) (layer "F.Cu") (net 11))
 (segment (start 162.4811 94.0436) (end 167.5611 99.1236) (width 0.1524) (layer "F.Cu") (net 11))
 (segment (start 162.3795 94.0944) (end 159.7887 94.0944) (width 0.1524) (layer "B.Cu") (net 11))
 (segment (start 159.7887 94.0944) (end 149.8827 104.0004) (width 0.1524) (layer "B.Cu") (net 11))
 (segment (start 149.8827 104.0004) (end 149.8827 105.372) (width 0.1524) (layer "B.Cu") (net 11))
 (segment (start 162.3795 94.0944) (end 162.4811 94.0436) (width 0.1524) (layer "B.Cu") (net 11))
 (segment (start 149.8827 105.372) (end 149.7811 105.4736) (width 0.1524) (layer "B.Cu") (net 11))
 (segment (start 152.3211 105.372) (end 144.7011 97.752) (width 0.1524) (layer "F.Cu") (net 10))
 (segment (start 152.3211 105.372) (end 152.3211 105.4736) (width 0.1524) (layer "F.Cu") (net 10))
 (segment (start 144.7011 97.752) (end 144.7011 94.0436) (width 0.1524) (layer "F.Cu") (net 10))
 (segment (start 156.1311 105.372) (end 167.5611 105.372) (width 0.1524) (layer "B.Cu") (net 10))
 (segment (start 167.5611 105.372) (end 167.5611 105.4736) (width 0.1524) (layer "B.Cu") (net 10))
 (segment (start 152.3211 105.372) (end 152.3211 105.4736) (width 0.1524) (layer "B.Cu") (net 10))
 (segment (start 152.3211 105.372) (end 153.2355 104.4576) (width 0.1524) (layer "B.Cu") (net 10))
 (segment (start 153.2355 104.4576) (end 155.2167 104.4576) (width 0.1524) (layer "B.Cu") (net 10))
 (segment (start 155.2167 104.4576) (end 156.1311 105.372) (width 0.1524) (layer "B.Cu") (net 10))
 (segment (start 154.9119 105.372) (end 154.8611 105.4736) (width 0.1524) (layer "F.Cu") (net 9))
 (segment (start 154.9119 100.3428) (end 154.9119 105.372) (width 0.1524) (layer "F.Cu") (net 9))
 (segment (start 156.1311 99.1236) (end 154.9119 100.3428) (width 0.1524) (layer "F.Cu") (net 9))
 (segment (start 157.3503 97.9044) (end 167.5611 97.9044) (width 0.1524) (layer "B.Cu") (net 9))
 (segment (start 156.1311 99.1236) (end 157.3503 97.9044) (width 0.1524) (layer "B.Cu") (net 9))
 (segment (start 167.5611 97.9044) (end 167.5611 97.8536) (width 0.1524) (layer "B.Cu") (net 9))
 (segment (start 161.3127 89.0652) (end 161.3127 99.1236) (width 0.1524) (layer "F.Cu") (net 8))
 (segment (start 161.3127 99.1236) (end 161.2111 99.1236) (width 0.1524) (layer "F.Cu") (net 8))
 (segment (start 161.3127 89.0652) (end 161.2111 88.9636) (width 0.1524) (layer "F.Cu") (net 8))
 (segment (start 163.7511 105.372) (end 151.1019 92.7228) (width 0.1524) (layer "F.Cu") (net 7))
 (segment (start 164.6655 109.0296) (end 164.6655 116.04) (width 0.1524) (layer "F.Cu") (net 7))
 (segment (start 164.6655 116.04) (end 159.0267 121.6788) (width 0.1524) (layer "F.Cu") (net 7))
 (segment (start 145.6155 121.6788) (end 144.7011 120.7644) (width 0.1524) (layer "F.Cu") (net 7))
 (segment (start 159.0267 121.6788) (end 145.6155 121.6788) (width 0.1524) (layer "F.Cu") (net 7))
 (segment (start 163.7511 108.1152) (end 164.6655 109.0296) (width 0.1524) (layer "F.Cu") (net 7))
 (segment (start 163.7511 108.0136) (end 163.7511 105.372) (width 0.1524) (layer "F.Cu") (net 7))
 (segment (start 151.1019 92.7228) (end 151.1019 91.5036) (width 0.1524) (layer "F.Cu") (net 7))
 (segment (start 140.8911 120.7644) (end 140.8911 120.7136) (width 0.1524) (layer "F.Cu") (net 7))
 (segment (start 153.5403 89.0652) (end 153.5911 88.9636) (width 0.1524) (layer "F.Cu") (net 7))
 (segment (start 163.7511 108.1152) (end 163.7511 108.0136) (width 0.1524) (layer "F.Cu") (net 7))
 (segment (start 153.5403 89.0652) (end 151.1019 91.5036) (width 0.1524) (layer "F.Cu") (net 7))
 (segment (start 151.1019 91.5036) (end 149.7811 91.5036) (width 0.1524) (layer "F.Cu") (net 7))
 (segment (start 144.7011 120.7644) (end 140.8911 120.7644) (width 0.1524) (layer "F.Cu") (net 7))
 (segment (start 157.3503 120.612) (end 157.4011 120.7136) (width 0.1524) (layer "F.Cu") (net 13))
 (segment (start 157.5027 120.612) (end 157.4011 120.7136) (width 0.1524) (layer "F.Cu") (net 13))
 (segment (start 163.7511 115.7352) (end 163.7511 115.6336) (width 0.1524) (layer "F.Cu") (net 13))
 (segment (start 158.8743 120.612) (end 157.5027 120.612) (width 0.1524) (layer "F.Cu") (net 13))
 (segment (start 163.7511 115.7352) (end 158.8743 120.612) (width 0.1524) (layer "F.Cu") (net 13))
 (segment (start 149.8827 113.1444) (end 149.7811 113.0936) (width 0.1524) (layer "F.Cu") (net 13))
 (segment (start 157.3503 120.612) (end 149.8827 113.1444) (width 0.1524) (layer "F.Cu") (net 13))
 (segment (start 149.8827 99.1236) (end 149.7811 99.1236) (width 0.1524) (layer "F.Cu") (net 14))
 (segment (start 153.2355 105.0672) (end 149.8827 101.7144) (width 0.1524) (layer "F.Cu") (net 14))
 (segment (start 153.2355 112.0776) (end 153.2355 105.0672) (width 0.1524) (layer "F.Cu") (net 14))
 (segment (start 152.3211 112.992) (end 152.3211 113.0936) (width 0.1524) (layer "F.Cu") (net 14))
 (segment (start 149.8827 101.7144) (end 149.8827 99.1236) (width 0.1524) (layer "F.Cu") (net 14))
 (segment (start 152.3211 112.992) (end 153.2355 112.0776) (width 0.1524) (layer "F.Cu") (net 14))
 (segment (start 152.3211 114.0588) (end 152.3211 120.7136) (width 0.1524) (layer "B.Cu") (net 14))
 (segment (start 156.1311 113.1444) (end 173.8095 113.1444) (width 0.1524) (layer "B.Cu") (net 14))
 (segment (start 152.3211 114.0588) (end 155.2167 114.0588) (width 0.1524) (layer "B.Cu") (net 14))
 (segment (start 173.8095 113.1444) (end 173.9111 113.0936) (width 0.1524) (layer "B.Cu") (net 14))
 (segment (start 155.2167 114.0588) (end 156.1311 113.1444) (width 0.1524) (layer "B.Cu") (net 14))
 (segment (start 152.3211 113.0936) (end 152.3211 114.0588) (width 0.1524) (layer "B.Cu") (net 14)))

